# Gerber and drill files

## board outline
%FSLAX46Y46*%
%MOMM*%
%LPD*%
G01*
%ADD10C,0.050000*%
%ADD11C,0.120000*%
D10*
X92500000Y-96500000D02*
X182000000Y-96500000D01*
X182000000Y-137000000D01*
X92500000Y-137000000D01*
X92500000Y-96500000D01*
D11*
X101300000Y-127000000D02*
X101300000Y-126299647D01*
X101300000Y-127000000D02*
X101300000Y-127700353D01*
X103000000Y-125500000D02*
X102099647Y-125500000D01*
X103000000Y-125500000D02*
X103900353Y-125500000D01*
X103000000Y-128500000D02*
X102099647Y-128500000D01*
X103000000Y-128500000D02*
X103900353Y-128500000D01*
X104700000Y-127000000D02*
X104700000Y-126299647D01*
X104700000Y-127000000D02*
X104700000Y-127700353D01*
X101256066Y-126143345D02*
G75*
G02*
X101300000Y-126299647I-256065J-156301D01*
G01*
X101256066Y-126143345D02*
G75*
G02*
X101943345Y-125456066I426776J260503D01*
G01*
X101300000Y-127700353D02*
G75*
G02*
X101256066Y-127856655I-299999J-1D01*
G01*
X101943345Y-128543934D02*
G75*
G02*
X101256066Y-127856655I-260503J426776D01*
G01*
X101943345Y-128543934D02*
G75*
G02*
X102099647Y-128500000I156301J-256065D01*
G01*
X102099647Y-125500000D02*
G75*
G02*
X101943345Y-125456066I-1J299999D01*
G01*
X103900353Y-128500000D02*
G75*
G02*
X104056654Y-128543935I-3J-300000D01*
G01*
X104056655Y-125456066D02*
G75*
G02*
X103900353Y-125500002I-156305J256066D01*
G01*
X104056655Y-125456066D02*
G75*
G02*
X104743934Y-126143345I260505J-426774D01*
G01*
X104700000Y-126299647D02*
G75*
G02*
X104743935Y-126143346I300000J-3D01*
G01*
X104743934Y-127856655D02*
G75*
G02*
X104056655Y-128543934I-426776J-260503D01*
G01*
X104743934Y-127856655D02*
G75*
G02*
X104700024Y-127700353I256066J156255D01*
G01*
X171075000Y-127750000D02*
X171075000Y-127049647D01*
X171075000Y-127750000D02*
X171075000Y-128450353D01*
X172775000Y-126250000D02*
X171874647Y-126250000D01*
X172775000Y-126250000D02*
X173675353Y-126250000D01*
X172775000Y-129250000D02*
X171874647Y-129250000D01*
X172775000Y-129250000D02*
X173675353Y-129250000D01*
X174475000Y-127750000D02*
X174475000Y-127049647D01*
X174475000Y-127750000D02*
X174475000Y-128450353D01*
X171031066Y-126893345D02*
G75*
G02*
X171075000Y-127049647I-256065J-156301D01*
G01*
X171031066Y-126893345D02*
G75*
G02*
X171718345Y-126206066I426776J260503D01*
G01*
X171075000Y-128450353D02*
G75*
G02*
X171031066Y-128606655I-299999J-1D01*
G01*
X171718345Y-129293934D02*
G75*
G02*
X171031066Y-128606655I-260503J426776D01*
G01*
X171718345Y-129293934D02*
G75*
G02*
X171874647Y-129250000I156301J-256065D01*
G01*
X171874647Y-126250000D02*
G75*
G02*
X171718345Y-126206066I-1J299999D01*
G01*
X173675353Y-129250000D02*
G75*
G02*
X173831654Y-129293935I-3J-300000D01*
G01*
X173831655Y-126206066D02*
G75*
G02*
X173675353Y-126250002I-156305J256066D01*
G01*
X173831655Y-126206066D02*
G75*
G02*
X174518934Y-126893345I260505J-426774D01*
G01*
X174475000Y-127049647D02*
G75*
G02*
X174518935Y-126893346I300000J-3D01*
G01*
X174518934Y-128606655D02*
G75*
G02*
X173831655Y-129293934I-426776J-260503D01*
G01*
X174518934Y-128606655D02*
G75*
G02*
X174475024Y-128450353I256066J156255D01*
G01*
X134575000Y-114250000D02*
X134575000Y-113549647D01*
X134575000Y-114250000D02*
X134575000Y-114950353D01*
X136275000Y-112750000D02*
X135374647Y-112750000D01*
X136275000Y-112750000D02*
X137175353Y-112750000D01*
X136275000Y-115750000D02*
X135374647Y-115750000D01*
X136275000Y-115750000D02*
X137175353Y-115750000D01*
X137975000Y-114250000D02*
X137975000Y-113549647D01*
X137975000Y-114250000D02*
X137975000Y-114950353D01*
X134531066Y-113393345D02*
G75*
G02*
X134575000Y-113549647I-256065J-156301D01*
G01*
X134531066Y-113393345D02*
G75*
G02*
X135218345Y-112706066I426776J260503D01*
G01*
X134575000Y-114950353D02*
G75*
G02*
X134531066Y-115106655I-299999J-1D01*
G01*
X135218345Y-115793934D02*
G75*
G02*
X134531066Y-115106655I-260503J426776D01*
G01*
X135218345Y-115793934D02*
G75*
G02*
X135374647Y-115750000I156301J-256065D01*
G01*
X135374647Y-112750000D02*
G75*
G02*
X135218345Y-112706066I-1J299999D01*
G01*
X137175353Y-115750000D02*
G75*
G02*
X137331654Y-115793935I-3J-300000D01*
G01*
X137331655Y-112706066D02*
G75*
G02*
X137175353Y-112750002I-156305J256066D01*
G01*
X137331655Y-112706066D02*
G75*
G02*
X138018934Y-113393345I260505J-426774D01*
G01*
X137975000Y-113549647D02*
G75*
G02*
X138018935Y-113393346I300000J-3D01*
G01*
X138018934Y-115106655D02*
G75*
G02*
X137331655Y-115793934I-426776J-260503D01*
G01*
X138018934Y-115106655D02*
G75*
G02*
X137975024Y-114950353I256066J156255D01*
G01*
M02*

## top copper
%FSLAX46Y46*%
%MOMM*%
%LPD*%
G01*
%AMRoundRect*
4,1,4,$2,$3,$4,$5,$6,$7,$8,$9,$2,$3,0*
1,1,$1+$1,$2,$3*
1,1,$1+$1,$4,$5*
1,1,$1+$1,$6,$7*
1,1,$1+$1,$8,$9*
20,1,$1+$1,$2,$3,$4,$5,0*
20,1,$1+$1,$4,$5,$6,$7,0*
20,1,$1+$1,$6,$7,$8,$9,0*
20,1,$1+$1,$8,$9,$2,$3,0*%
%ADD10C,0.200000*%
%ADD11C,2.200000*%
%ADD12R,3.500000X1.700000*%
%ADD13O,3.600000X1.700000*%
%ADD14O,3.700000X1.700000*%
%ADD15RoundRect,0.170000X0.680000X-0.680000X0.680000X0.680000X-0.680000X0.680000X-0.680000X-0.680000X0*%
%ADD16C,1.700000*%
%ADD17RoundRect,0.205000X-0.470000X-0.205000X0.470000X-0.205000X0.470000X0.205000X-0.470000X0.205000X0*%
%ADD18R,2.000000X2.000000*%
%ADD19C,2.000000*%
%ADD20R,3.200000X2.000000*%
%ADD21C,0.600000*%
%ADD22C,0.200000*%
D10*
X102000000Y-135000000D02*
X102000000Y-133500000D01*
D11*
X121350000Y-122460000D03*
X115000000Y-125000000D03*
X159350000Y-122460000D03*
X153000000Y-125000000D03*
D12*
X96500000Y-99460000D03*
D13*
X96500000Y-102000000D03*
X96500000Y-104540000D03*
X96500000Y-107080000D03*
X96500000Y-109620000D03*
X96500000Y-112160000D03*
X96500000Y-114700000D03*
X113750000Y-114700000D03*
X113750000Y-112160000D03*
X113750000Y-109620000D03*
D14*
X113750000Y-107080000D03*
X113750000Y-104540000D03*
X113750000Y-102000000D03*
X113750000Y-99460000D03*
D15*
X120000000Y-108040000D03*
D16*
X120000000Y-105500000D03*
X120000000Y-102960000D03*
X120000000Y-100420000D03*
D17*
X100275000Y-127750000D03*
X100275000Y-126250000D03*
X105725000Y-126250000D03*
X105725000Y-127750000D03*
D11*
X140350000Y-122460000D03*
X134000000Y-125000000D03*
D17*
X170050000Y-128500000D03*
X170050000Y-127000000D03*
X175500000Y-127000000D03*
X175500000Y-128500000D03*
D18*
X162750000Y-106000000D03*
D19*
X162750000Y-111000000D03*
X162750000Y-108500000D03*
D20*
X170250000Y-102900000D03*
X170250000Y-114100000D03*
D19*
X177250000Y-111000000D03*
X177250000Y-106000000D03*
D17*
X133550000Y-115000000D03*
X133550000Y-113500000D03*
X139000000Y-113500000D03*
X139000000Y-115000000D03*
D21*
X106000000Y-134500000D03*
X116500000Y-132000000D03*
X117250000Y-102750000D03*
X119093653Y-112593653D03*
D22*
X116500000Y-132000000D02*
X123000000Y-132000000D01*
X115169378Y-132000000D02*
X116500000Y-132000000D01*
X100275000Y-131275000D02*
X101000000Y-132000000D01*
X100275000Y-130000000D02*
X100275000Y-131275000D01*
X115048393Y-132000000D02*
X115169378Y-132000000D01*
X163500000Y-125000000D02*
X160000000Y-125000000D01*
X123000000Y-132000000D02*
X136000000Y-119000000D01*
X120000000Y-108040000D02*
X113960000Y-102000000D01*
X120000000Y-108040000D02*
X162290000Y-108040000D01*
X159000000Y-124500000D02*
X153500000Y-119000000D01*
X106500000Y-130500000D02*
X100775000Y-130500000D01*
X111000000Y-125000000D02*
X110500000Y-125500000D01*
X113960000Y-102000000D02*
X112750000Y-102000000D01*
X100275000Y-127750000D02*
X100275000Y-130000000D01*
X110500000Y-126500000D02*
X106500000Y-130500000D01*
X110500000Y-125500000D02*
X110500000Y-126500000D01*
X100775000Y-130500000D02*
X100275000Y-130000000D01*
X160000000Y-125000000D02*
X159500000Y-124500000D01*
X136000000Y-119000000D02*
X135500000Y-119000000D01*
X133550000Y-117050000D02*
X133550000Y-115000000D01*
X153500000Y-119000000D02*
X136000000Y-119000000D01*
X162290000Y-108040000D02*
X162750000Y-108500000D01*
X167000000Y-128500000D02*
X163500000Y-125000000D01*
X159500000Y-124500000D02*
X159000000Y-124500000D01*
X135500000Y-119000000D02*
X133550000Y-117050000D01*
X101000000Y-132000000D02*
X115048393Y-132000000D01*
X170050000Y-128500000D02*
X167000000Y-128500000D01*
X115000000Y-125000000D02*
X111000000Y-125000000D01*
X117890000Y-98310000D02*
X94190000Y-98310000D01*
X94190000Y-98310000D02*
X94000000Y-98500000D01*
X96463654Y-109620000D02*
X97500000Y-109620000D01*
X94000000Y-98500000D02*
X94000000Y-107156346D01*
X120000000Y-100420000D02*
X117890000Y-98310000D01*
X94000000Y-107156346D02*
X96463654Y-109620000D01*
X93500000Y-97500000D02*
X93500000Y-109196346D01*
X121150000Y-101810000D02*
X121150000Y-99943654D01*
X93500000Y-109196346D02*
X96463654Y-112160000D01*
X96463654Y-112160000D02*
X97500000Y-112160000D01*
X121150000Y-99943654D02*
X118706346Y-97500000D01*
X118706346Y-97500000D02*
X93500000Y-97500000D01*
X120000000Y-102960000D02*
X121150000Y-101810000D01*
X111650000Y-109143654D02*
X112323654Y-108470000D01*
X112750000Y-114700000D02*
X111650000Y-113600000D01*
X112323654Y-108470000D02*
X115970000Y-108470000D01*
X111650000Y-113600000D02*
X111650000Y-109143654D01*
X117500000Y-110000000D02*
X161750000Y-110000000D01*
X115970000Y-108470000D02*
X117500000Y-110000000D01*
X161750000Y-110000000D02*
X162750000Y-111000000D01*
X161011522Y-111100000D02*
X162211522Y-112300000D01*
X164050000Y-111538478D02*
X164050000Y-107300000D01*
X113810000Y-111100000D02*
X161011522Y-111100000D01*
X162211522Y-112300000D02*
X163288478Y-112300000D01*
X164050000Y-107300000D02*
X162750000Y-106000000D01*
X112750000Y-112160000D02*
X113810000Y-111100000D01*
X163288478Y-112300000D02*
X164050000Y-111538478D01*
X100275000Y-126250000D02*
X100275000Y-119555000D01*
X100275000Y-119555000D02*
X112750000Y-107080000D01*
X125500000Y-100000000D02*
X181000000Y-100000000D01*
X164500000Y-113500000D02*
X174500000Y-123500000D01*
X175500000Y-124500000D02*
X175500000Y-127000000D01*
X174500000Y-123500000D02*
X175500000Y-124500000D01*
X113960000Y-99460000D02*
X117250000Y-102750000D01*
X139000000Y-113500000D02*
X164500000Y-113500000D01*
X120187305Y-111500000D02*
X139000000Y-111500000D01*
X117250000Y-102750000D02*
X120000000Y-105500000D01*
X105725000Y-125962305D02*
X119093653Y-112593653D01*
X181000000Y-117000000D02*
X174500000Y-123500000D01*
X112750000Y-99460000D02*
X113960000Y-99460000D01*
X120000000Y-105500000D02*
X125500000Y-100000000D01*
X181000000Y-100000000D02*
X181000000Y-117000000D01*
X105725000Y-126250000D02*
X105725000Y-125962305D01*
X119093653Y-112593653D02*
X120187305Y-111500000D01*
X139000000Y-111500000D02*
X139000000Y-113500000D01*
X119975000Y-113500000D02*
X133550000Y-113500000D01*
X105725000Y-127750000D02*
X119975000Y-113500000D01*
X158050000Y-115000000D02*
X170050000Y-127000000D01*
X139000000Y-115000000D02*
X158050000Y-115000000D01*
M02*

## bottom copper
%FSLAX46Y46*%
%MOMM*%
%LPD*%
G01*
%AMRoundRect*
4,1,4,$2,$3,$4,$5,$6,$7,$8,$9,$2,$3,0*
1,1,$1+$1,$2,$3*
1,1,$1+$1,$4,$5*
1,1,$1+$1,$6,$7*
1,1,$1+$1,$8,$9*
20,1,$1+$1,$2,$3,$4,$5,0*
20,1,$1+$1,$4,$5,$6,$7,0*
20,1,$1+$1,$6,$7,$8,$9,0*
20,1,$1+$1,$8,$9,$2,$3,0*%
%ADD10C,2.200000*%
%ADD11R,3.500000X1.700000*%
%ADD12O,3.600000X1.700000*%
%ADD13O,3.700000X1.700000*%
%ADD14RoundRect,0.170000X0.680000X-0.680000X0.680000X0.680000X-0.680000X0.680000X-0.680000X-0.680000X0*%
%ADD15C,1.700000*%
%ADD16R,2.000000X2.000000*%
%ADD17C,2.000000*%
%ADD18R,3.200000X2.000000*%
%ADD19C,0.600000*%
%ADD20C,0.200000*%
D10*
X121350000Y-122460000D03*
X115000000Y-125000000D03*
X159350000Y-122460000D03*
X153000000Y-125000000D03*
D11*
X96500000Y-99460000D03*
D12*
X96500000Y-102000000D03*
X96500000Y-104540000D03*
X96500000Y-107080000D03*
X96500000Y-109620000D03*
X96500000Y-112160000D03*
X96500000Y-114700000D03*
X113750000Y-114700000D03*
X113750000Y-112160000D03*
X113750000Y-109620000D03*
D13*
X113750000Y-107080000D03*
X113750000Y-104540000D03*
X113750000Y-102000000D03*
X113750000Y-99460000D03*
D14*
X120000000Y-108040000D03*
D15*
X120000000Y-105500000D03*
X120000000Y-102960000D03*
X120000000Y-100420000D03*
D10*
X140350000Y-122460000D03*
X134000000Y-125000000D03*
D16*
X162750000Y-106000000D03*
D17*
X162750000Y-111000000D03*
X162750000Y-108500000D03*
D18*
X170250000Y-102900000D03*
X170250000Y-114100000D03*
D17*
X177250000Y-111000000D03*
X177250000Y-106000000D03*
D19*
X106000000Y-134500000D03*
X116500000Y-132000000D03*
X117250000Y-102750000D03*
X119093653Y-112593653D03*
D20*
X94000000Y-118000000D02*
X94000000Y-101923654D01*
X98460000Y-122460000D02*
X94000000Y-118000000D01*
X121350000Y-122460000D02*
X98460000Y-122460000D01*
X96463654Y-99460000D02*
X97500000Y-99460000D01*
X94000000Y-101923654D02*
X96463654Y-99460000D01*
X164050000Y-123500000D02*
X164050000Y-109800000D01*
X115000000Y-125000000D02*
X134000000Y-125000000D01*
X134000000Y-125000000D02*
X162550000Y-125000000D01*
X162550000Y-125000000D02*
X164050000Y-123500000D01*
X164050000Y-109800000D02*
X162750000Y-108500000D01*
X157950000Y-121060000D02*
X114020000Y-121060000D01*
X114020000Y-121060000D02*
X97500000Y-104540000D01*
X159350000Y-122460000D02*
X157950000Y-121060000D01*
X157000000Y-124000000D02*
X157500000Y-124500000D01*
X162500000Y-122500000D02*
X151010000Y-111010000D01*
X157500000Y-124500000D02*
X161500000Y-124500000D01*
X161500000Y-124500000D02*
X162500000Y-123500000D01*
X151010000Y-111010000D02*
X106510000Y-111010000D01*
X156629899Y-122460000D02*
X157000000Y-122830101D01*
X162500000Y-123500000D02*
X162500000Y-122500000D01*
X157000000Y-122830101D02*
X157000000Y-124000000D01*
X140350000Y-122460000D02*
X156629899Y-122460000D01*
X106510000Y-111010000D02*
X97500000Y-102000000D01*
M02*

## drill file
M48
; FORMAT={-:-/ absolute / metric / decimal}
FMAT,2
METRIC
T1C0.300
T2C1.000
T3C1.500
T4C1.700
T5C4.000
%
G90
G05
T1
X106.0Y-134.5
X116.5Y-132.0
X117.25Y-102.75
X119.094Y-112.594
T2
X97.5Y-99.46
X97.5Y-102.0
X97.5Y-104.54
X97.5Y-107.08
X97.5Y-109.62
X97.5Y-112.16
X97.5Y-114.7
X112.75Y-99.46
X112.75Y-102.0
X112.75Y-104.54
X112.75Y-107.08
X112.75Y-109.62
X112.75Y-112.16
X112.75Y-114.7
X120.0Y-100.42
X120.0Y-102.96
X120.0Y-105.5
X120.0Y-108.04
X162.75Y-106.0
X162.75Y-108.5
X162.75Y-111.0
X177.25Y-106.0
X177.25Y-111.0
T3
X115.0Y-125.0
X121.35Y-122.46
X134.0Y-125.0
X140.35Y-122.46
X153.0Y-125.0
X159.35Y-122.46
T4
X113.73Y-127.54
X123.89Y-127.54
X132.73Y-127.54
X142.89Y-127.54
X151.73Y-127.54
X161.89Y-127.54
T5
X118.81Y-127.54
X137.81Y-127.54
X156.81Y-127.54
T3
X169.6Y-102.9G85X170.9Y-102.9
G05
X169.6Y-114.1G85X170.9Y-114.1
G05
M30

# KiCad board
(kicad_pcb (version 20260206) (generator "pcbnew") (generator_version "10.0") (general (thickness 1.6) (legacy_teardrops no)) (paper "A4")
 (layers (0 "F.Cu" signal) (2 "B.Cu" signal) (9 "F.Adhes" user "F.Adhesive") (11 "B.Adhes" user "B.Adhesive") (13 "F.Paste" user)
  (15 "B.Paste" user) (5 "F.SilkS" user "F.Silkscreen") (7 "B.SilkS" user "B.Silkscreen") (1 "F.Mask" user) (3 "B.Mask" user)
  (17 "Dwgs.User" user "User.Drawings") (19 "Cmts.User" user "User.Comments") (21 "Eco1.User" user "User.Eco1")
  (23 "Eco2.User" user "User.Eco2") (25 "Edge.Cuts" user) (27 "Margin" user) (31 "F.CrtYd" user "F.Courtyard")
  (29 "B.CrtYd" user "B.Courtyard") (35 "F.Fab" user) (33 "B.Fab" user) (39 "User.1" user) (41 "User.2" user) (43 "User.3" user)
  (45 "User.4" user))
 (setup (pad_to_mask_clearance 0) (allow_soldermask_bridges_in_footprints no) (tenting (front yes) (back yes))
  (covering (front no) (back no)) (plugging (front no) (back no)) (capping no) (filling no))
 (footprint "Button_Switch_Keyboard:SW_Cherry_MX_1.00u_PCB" (layer "F.Cu") (at 121.35 122.46)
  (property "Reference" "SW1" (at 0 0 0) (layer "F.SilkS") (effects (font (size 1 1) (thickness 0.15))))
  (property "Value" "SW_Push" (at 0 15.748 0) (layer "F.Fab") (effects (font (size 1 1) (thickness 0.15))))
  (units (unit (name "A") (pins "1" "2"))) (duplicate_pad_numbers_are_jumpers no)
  (pad "" np_thru_hole circle (at -7.62 5.08) (size 1.7 1.7) (drill 1.7) (layers "*.Cu" "*.Mask"))
  (pad "" np_thru_hole circle (at -2.54 5.08) (size 4 4) (drill 4) (layers "*.Cu" "*.Mask"))
  (pad "" np_thru_hole circle (at 2.54 5.08) (size 1.7 1.7) (drill 1.7) (layers "*.Cu" "*.Mask"))
  (pad "1" thru_hole circle (at 0 0) (size 2.2 2.2) (drill 1.5) (layers "*.Cu" "*.Mask") (remove_unused_layers no)
   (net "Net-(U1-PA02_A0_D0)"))
  (pad "2" thru_hole circle (at -6.35 2.54) (size 2.2 2.2) (drill 1.5) (layers "*.Cu" "*.Mask") (remove_unused_layers no) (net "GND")))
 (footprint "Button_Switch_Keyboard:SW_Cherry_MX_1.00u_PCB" (layer "F.Cu") (at 159.35 122.46)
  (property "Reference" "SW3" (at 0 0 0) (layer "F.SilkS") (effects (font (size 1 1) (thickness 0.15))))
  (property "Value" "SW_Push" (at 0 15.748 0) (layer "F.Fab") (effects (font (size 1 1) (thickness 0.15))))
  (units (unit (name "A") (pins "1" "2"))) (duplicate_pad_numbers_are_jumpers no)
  (pad "" np_thru_hole circle (at -7.62 5.08) (size 1.7 1.7) (drill 1.7) (layers "*.Cu" "*.Mask"))
  (pad "" np_thru_hole circle (at -2.54 5.08) (size 4 4) (drill 4) (layers "*.Cu" "*.Mask"))
  (pad "" np_thru_hole circle (at 2.54 5.08) (size 1.7 1.7) (drill 1.7) (layers "*.Cu" "*.Mask"))
  (pad "1" thru_hole circle (at 0 0) (size 2.2 2.2) (drill 1.5) (layers "*.Cu" "*.Mask") (remove_unused_layers no)
   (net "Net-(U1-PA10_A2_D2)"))
  (pad "2" thru_hole circle (at -6.35 2.54) (size 2.2 2.2) (drill 1.5) (layers "*.Cu" "*.Mask") (remove_unused_layers no) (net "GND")))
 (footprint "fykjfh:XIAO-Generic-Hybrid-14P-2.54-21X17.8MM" (layer "F.Cu") (at 105.125 107.08)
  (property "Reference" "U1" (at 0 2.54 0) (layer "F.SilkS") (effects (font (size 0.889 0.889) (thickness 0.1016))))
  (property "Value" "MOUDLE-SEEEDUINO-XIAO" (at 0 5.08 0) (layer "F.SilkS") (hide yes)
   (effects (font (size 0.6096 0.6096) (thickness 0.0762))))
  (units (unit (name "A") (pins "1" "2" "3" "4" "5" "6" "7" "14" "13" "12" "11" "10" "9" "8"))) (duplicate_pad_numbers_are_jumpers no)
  (pad "1" thru_hole rect (at -7.625 -7.62) (size 3.5 1.7) (drill 1 (offset -1 0)) (layers "*.Cu" "*.Mask") (remove_unused_layers no)
   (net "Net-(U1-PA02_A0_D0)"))
  (pad "2" thru_hole oval (at -7.625 -5.08) (size 3.6 1.7) (drill 1 (offset -1 0)) (layers "*.Cu" "*.Mask") (remove_unused_layers no)
   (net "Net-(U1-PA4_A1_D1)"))
  (pad "3" thru_hole oval (at -7.625 -2.54) (size 3.6 1.7) (drill 1 (offset -1 0)) (layers "*.Cu" "*.Mask") (remove_unused_layers no)
   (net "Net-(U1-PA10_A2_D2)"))
  (pad "4" thru_hole oval (at -7.625 0) (size 3.6 1.7) (drill 1 (offset -1 0)) (layers "*.Cu" "*.Mask") (remove_unused_layers no)
   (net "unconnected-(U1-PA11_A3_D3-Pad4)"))
  (pad "5" thru_hole oval (at -7.625 2.54) (size 3.6 1.7) (drill 1 (offset -1 0)) (layers "*.Cu" "*.Mask") (remove_unused_layers no)
   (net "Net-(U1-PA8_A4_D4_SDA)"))
  (pad "6" thru_hole oval (at -7.625 5.08 180) (size 3.6 1.7) (drill 1 (offset 1 0)) (layers "*.Cu" "*.Mask") (remove_unused_layers no)
   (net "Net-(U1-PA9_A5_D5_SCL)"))
  (pad "7" thru_hole oval (at -7.625 7.62) (size 3.6 1.7) (drill 1 (offset -1 0)) (layers "*.Cu" "*.Mask") (remove_unused_layers no)
   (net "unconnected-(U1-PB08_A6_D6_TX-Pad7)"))
  (pad "8" thru_hole oval (at 7.625 7.62) (size 3.6 1.7) (drill 1 (offset 1 0)) (layers "*.Cu" "*.Mask") (remove_unused_layers no)
   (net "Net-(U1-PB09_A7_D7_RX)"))
  (pad "9" thru_hole oval (at 7.625 5.08) (size 3.6 1.7) (drill 1 (offset 1 0)) (layers "*.Cu" "*.Mask") (remove_unused_layers no)
   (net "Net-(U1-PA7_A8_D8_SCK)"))
  (pad "10" thru_hole oval (at 7.625 2.54) (size 3.6 1.7) (drill 1 (offset 1 0)) (layers "*.Cu" "*.Mask") (remove_unused_layers no)
   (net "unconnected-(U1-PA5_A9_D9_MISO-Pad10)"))
  (pad "11" thru_hole oval (at 7.625 0) (size 3.7 1.7) (drill 1 (offset 1 0)) (layers "*.Cu" "*.Mask") (remove_unused_layers no)
   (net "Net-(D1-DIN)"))
  (pad "12" thru_hole oval (at 7.625 -2.54) (size 3.7 1.7) (drill 1 (offset 1 0)) (layers "*.Cu" "*.Mask") (remove_unused_layers no)
   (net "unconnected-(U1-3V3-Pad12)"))
  (pad "13" thru_hole oval (at 7.625 -5.08) (size 3.7 1.7) (drill 1 (offset 1 0)) (layers "*.Cu" "*.Mask") (remove_unused_layers no)
   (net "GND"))
  (pad "14" thru_hole oval (at 7.625 -7.62) (size 3.7 1.7) (drill 1 (offset 1 0)) (layers "*.Cu" "*.Mask") (remove_unused_layers no)
   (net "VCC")))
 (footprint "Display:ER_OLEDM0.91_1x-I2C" (layer "F.Cu") (at 120 108.04 90)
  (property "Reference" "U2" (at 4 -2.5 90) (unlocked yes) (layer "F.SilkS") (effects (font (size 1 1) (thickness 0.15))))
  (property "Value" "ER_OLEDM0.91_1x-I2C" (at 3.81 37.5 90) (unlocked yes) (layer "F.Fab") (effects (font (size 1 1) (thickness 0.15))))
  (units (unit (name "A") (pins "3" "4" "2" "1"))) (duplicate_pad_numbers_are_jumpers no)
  (pad "1" thru_hole roundrect (at 0 0 90) (size 1.7 1.7) (drill 1) (layers "*.Cu" "*.Mask") (remove_unused_layers no)
   (roundrect_rratio 0.1) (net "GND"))
  (pad "2" thru_hole circle (at 2.54 0 90) (size 1.7 1.7) (drill 1) (layers "*.Cu" "*.Mask") (remove_unused_layers no) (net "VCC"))
  (pad "3" thru_hole circle (at 5.08 0 90) (size 1.7 1.7) (drill 1) (layers "*.Cu" "*.Mask") (remove_unused_layers no)
   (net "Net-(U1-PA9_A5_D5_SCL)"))
  (pad "4" thru_hole circle (at 7.62 0 90) (size 1.7 1.7) (drill 1) (layers "*.Cu" "*.Mask") (remove_unused_layers no)
   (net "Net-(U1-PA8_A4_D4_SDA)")))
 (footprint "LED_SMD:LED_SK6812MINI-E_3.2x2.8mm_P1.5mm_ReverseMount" (layer "F.Cu") (at 103 127)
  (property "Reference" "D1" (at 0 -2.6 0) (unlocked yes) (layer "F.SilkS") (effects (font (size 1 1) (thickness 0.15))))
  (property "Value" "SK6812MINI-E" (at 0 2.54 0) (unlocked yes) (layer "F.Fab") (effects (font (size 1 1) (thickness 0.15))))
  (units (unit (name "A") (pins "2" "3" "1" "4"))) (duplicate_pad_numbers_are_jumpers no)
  (fp_line (start -1.7 0) (end -1.7 -0.700353) (stroke (width 0.12) (type solid)) (layer "Edge.Cuts"))
  (fp_line (start -1.7 0) (end -1.7 0.700353) (stroke (width 0.12) (type solid)) (layer "Edge.Cuts"))
  (fp_line (start 0 -1.5) (end -0.900353 -1.5) (stroke (width 0.12) (type solid)) (layer "Edge.Cuts"))
  (fp_line (start 0 -1.5) (end 0.900353 -1.5) (stroke (width 0.12) (type solid)) (layer "Edge.Cuts"))
  (fp_line (start 0 1.5) (end -0.900353 1.5) (stroke (width 0.12) (type solid)) (layer "Edge.Cuts"))
  (fp_line (start 0 1.5) (end 0.900353 1.5) (stroke (width 0.12) (type solid)) (layer "Edge.Cuts"))
  (fp_line (start 1.7 0) (end 1.7 -0.700353) (stroke (width 0.12) (type solid)) (layer "Edge.Cuts"))
  (fp_line (start 1.7 0) (end 1.7 0.700353) (stroke (width 0.12) (type solid)) (layer "Edge.Cuts"))
  (fp_arc (start -1.743934 -0.856655) (mid -1.711192 -0.781532) (end -1.7 -0.700353) (stroke (width 0.12) (type solid)) (layer "Edge.Cuts"))
  (fp_arc (start -1.743934 -0.856655) (mid -1.670711 -1.470711) (end -1.056655 -1.543934) (stroke (width 0.12) (type solid))
   (layer "Edge.Cuts"))
  (fp_arc (start -1.7 0.700353) (mid -1.711192 0.781532) (end -1.743934 0.856655) (stroke (width 0.12) (type solid)) (layer "Edge.Cuts"))
  (fp_arc (start -1.056655 1.543934) (mid -1.670711 1.470711) (end -1.743934 0.856655) (stroke (width 0.12) (type solid))
   (layer "Edge.Cuts"))
  (fp_arc (start -1.056655 1.543934) (mid -0.981532 1.511192) (end -0.900353 1.5) (stroke (width 0.12) (type solid)) (layer "Edge.Cuts"))
  (fp_arc (start -0.900353 -1.5) (mid -0.981532 -1.511192) (end -1.056655 -1.543934) (stroke (width 0.12) (type solid)) (layer "Edge.Cuts"))
  (fp_arc (start 0.900353 1.5) (mid 0.981532 1.511192) (end 1.056655 1.543934) (stroke (width 0.12) (type solid)) (layer "Edge.Cuts"))
  (fp_arc (start 1.056655 -1.543934) (mid 0.981532 -1.511192) (end 0.900353 -1.5) (stroke (width 0.12) (type solid)) (layer "Edge.Cuts"))
  (fp_arc (start 1.056655 -1.543934) (mid 1.670711 -1.470711) (end 1.743934 -0.856655) (stroke (width 0.12) (type solid))
   (layer "Edge.Cuts"))
  (fp_arc (start 1.7 -0.700353) (mid 1.711192 -0.781532) (end 1.743934 -0.856655) (stroke (width 0.12) (type solid)) (layer "Edge.Cuts"))
  (fp_arc (start 1.743934 0.856655) (mid 1.670711 1.470711) (end 1.056655 1.543934) (stroke (width 0.12) (type solid)) (layer "Edge.Cuts"))
  (fp_arc (start 1.743934 0.856655) (mid 1.711192 0.781532) (end 1.7 0.700353) (stroke (width 0.12) (type solid)) (layer "Edge.Cuts"))
  (pad "1" smd roundrect (at -2.725 0.75) (size 1.35 0.82) (layers "F.Cu" "F.Mask" "F.Paste") (roundrect_rratio 0.25) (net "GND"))
  (pad "2" smd roundrect (at -2.725 -0.75) (size 1.35 0.82) (layers "F.Cu" "F.Mask" "F.Paste") (roundrect_rratio 0.25) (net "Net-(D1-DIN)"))
  (pad "3" smd roundrect (at 2.725 -0.75) (size 1.35 0.82) (layers "F.Cu" "F.Mask" "F.Paste") (roundrect_rratio 0.25) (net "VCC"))
  (pad "4" smd roundrect (at 2.725 0.75) (size 1.35 0.82) (layers "F.Cu" "F.Mask" "F.Paste") (roundrect_rratio 0.25) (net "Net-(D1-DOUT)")))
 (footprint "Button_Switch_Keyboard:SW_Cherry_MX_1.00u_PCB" (layer "F.Cu") (at 140.35 122.46)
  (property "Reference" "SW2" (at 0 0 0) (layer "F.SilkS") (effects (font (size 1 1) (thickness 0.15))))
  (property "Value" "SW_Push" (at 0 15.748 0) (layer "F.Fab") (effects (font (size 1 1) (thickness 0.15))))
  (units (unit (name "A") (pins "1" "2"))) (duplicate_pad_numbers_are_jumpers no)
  (pad "" np_thru_hole circle (at -7.62 5.08) (size 1.7 1.7) (drill 1.7) (layers "*.Cu" "*.Mask"))
  (pad "" np_thru_hole circle (at -2.54 5.08) (size 4 4) (drill 4) (layers "*.Cu" "*.Mask"))
  (pad "" np_thru_hole circle (at 2.54 5.08) (size 1.7 1.7) (drill 1.7) (layers "*.Cu" "*.Mask"))
  (pad "1" thru_hole circle (at 0 0) (size 2.2 2.2) (drill 1.5) (layers "*.Cu" "*.Mask") (remove_unused_layers no)
   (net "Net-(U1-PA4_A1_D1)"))
  (pad "2" thru_hole circle (at -6.35 2.54) (size 2.2 2.2) (drill 1.5) (layers "*.Cu" "*.Mask") (remove_unused_layers no) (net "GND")))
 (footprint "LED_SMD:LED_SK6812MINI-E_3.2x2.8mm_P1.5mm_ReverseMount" (layer "F.Cu") (at 172.775 127.75)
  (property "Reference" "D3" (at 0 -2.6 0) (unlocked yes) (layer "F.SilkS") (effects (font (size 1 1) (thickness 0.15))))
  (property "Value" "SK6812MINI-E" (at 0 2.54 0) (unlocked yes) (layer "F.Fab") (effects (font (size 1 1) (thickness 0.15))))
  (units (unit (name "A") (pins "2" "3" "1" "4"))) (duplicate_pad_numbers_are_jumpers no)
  (fp_line (start -1.7 0) (end -1.7 -0.700353) (stroke (width 0.12) (type solid)) (layer "Edge.Cuts"))
  (fp_line (start -1.7 0) (end -1.7 0.700353) (stroke (width 0.12) (type solid)) (layer "Edge.Cuts"))
  (fp_line (start 0 -1.5) (end -0.900353 -1.5) (stroke (width 0.12) (type solid)) (layer "Edge.Cuts"))
  (fp_line (start 0 -1.5) (end 0.900353 -1.5) (stroke (width 0.12) (type solid)) (layer "Edge.Cuts"))
  (fp_line (start 0 1.5) (end -0.900353 1.5) (stroke (width 0.12) (type solid)) (layer "Edge.Cuts"))
  (fp_line (start 0 1.5) (end 0.900353 1.5) (stroke (width 0.12) (type solid)) (layer "Edge.Cuts"))
  (fp_line (start 1.7 0) (end 1.7 -0.700353) (stroke (width 0.12) (type solid)) (layer "Edge.Cuts"))
  (fp_line (start 1.7 0) (end 1.7 0.700353) (stroke (width 0.12) (type solid)) (layer "Edge.Cuts"))
  (fp_arc (start -1.743934 -0.856655) (mid -1.711192 -0.781532) (end -1.7 -0.700353) (stroke (width 0.12) (type solid)) (layer "Edge.Cuts"))
  (fp_arc (start -1.743934 -0.856655) (mid -1.670711 -1.470711) (end -1.056655 -1.543934) (stroke (width 0.12) (type solid))
   (layer "Edge.Cuts"))
  (fp_arc (start -1.7 0.700353) (mid -1.711192 0.781532) (end -1.743934 0.856655) (stroke (width 0.12) (type solid)) (layer "Edge.Cuts"))
  (fp_arc (start -1.056655 1.543934) (mid -1.670711 1.470711) (end -1.743934 0.856655) (stroke (width 0.12) (type solid))
   (layer "Edge.Cuts"))
  (fp_arc (start -1.056655 1.543934) (mid -0.981532 1.511192) (end -0.900353 1.5) (stroke (width 0.12) (type solid)) (layer "Edge.Cuts"))
  (fp_arc (start -0.900353 -1.5) (mid -0.981532 -1.511192) (end -1.056655 -1.543934) (stroke (width 0.12) (type solid)) (layer "Edge.Cuts"))
  (fp_arc (start 0.900353 1.5) (mid 0.981532 1.511192) (end 1.056655 1.543934) (stroke (width 0.12) (type solid)) (layer "Edge.Cuts"))
  (fp_arc (start 1.056655 -1.543934) (mid 0.981532 -1.511192) (end 0.900353 -1.5) (stroke (width 0.12) (type solid)) (layer "Edge.Cuts"))
  (fp_arc (start 1.056655 -1.543934) (mid 1.670711 -1.470711) (end 1.743934 -0.856655) (stroke (width 0.12) (type solid))
   (layer "Edge.Cuts"))
  (fp_arc (start 1.7 -0.700353) (mid 1.711192 -0.781532) (end 1.743934 -0.856655) (stroke (width 0.12) (type solid)) (layer "Edge.Cuts"))
  (fp_arc (start 1.743934 0.856655) (mid 1.670711 1.470711) (end 1.056655 1.543934) (stroke (width 0.12) (type solid)) (layer "Edge.Cuts"))
  (fp_arc (start 1.743934 0.856655) (mid 1.711192 0.781532) (end 1.7 0.700353) (stroke (width 0.12) (type solid)) (layer "Edge.Cuts"))
  (pad "1" smd roundrect (at -2.725 0.75) (size 1.35 0.82) (layers "F.Cu" "F.Mask" "F.Paste") (roundrect_rratio 0.25) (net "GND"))
  (pad "2" smd roundrect (at -2.725 -0.75) (size 1.35 0.82) (layers "F.Cu" "F.Mask" "F.Paste") (roundrect_rratio 0.25) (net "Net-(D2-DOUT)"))
  (pad "3" smd roundrect (at 2.725 -0.75) (size 1.35 0.82) (layers "F.Cu" "F.Mask" "F.Paste") (roundrect_rratio 0.25) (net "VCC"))
  (pad "4" smd roundrect (at 2.725 0.75) (size 1.35 0.82) (layers "F.Cu" "F.Mask" "F.Paste") (roundrect_rratio 0.25)
   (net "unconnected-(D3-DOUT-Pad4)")))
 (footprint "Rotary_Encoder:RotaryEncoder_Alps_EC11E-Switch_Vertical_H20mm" (layer "F.Cu") (at 162.75 106)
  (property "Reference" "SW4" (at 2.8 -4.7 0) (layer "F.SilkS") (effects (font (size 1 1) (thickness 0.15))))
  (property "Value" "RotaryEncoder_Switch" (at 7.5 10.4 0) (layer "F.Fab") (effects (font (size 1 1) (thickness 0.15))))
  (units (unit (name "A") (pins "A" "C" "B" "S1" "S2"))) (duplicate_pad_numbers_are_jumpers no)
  (pad "A" thru_hole rect (at 0 0) (size 2 2) (drill 1) (layers "*.Cu" "*.Mask") (remove_unused_layers no) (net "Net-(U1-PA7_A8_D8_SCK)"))
  (pad "B" thru_hole circle (at 0 5) (size 2 2) (drill 1) (layers "*.Cu" "*.Mask") (remove_unused_layers no) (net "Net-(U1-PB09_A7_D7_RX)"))
  (pad "C" thru_hole circle (at 0 2.5) (size 2 2) (drill 1) (layers "*.Cu" "*.Mask") (remove_unused_layers no) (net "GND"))
  (pad "MP" thru_hole rect (at 7.5 -3.1) (size 3.2 2) (drill oval 2.8 1.5) (layers "*.Cu" "*.Mask") (remove_unused_layers no))
  (pad "MP" thru_hole rect (at 7.5 8.1) (size 3.2 2) (drill oval 2.8 1.5) (layers "*.Cu" "*.Mask") (remove_unused_layers no))
  (pad "S1" thru_hole circle (at 14.5 5) (size 2 2) (drill 1) (layers "*.Cu" "*.Mask") (remove_unused_layers no)
   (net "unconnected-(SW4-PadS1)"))
  (pad "S2" thru_hole circle (at 14.5 0) (size 2 2) (drill 1) (layers "*.Cu" "*.Mask") (remove_unused_layers no)
   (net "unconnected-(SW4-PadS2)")))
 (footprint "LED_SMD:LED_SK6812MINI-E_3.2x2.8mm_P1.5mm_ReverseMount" (layer "F.Cu") (at 136.275 114.25)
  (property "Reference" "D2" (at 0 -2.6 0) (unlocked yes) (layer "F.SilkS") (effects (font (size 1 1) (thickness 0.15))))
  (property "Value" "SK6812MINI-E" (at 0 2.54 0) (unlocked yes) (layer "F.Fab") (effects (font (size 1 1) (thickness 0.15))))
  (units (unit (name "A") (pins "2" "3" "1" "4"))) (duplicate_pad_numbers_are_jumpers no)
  (fp_line (start -1.7 0) (end -1.7 -0.700353) (stroke (width 0.12) (type solid)) (layer "Edge.Cuts"))
  (fp_line (start -1.7 0) (end -1.7 0.700353) (stroke (width 0.12) (type solid)) (layer "Edge.Cuts"))
  (fp_line (start 0 -1.5) (end -0.900353 -1.5) (stroke (width 0.12) (type solid)) (layer "Edge.Cuts"))
  (fp_line (start 0 -1.5) (end 0.900353 -1.5) (stroke (width 0.12) (type solid)) (layer "Edge.Cuts"))
  (fp_line (start 0 1.5) (end -0.900353 1.5) (stroke (width 0.12) (type solid)) (layer "Edge.Cuts"))
  (fp_line (start 0 1.5) (end 0.900353 1.5) (stroke (width 0.12) (type solid)) (layer "Edge.Cuts"))
  (fp_line (start 1.7 0) (end 1.7 -0.700353) (stroke (width 0.12) (type solid)) (layer "Edge.Cuts"))
  (fp_line (start 1.7 0) (end 1.7 0.700353) (stroke (width 0.12) (type solid)) (layer "Edge.Cuts"))
  (fp_arc (start -1.743934 -0.856655) (mid -1.711192 -0.781532) (end -1.7 -0.700353) (stroke (width 0.12) (type solid)) (layer "Edge.Cuts"))
  (fp_arc (start -1.743934 -0.856655) (mid -1.670711 -1.470711) (end -1.056655 -1.543934) (stroke (width 0.12) (type solid))
   (layer "Edge.Cuts"))
  (fp_arc (start -1.7 0.700353) (mid -1.711192 0.781532) (end -1.743934 0.856655) (stroke (width 0.12) (type solid)) (layer "Edge.Cuts"))
  (fp_arc (start -1.056655 1.543934) (mid -1.670711 1.470711) (end -1.743934 0.856655) (stroke (width 0.12) (type solid))
   (layer "Edge.Cuts"))
  (fp_arc (start -1.056655 1.543934) (mid -0.981532 1.511192) (end -0.900353 1.5) (stroke (width 0.12) (type solid)) (layer "Edge.Cuts"))
  (fp_arc (start -0.900353 -1.5) (mid -0.981532 -1.511192) (end -1.056655 -1.543934) (stroke (width 0.12) (type solid)) (layer "Edge.Cuts"))
  (fp_arc (start 0.900353 1.5) (mid 0.981532 1.511192) (end 1.056655 1.543934) (stroke (width 0.12) (type solid)) (layer "Edge.Cuts"))
  (fp_arc (start 1.056655 -1.543934) (mid 0.981532 -1.511192) (end 0.900353 -1.5) (stroke (width 0.12) (type solid)) (layer "Edge.Cuts"))
  (fp_arc (start 1.056655 -1.543934) (mid 1.670711 -1.470711) (end 1.743934 -0.856655) (stroke (width 0.12) (type solid))
   (layer "Edge.Cuts"))
  (fp_arc (start 1.7 -0.700353) (mid 1.711192 -0.781532) (end 1.743934 -0.856655) (stroke (width 0.12) (type solid)) (layer "Edge.Cuts"))
  (fp_arc (start 1.743934 0.856655) (mid 1.670711 1.470711) (end 1.056655 1.543934) (stroke (width 0.12) (type solid)) (layer "Edge.Cuts"))
  (fp_arc (start 1.743934 0.856655) (mid 1.711192 0.781532) (end 1.7 0.700353) (stroke (width 0.12) (type solid)) (layer "Edge.Cuts"))
  (pad "1" smd roundrect (at -2.725 0.75) (size 1.35 0.82) (layers "F.Cu" "F.Mask" "F.Paste") (roundrect_rratio 0.25) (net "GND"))
  (pad "2" smd roundrect (at -2.725 -0.75) (size 1.35 0.82) (layers "F.Cu" "F.Mask" "F.Paste") (roundrect_rratio 0.25) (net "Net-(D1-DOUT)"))
  (pad "3" smd roundrect (at 2.725 -0.75) (size 1.35 0.82) (layers "F.Cu" "F.Mask" "F.Paste") (roundrect_rratio 0.25) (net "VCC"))
  (pad "4" smd roundrect (at 2.725 0.75) (size 1.35 0.82) (layers "F.Cu" "F.Mask" "F.Paste") (roundrect_rratio 0.25) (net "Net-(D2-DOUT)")))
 (gr_line (start 102 135) (end 102 133.5) (stroke (width 0.2) (type default)) (layer "F.Cu"))
 (gr_rect (start 92.5 96.5) (end 182 137) (stroke (width 0.05) (type default)) (fill no) (layer "Edge.Cuts"))
 (via (at 106 134.5) (size 0.6) (drill 0.3) (layers "F.Cu" "B.Cu") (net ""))
 (segment (start 94 118) (end 94 101.923654) (width 0.2) (layer "B.Cu") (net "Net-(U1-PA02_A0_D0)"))
 (segment (start 98.46 122.46) (end 94 118) (width 0.2) (layer "B.Cu") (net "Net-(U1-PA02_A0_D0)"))
 (segment (start 121.35 122.46) (end 98.46 122.46) (width 0.2) (layer "B.Cu") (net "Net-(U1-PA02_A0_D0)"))
 (segment (start 96.463654 99.46) (end 97.5 99.46) (width 0.2) (layer "B.Cu") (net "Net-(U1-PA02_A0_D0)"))
 (segment (start 94 101.923654) (end 96.463654 99.46) (width 0.2) (layer "B.Cu") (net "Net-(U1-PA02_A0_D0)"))
 (segment (start 116.5 132) (end 123 132) (width 0.2) (layer "F.Cu") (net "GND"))
 (segment (start 115.169378 132) (end 116.5 132) (width 0.2) (layer "F.Cu") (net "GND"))
 (segment (start 100.275 131.275) (end 101 132) (width 0.2) (layer "F.Cu") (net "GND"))
 (segment (start 100.275 130) (end 100.275 131.275) (width 0.2) (layer "F.Cu") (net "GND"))
 (segment (start 115.048393 132) (end 115.169378 132) (width 0.2) (layer "F.Cu") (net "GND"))
 (segment (start 163.5 125) (end 160 125) (width 0.2) (layer "F.Cu") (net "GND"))
 (segment (start 123 132) (end 136 119) (width 0.2) (layer "F.Cu") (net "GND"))
 (segment (start 120 108.04) (end 113.96 102) (width 0.2) (layer "F.Cu") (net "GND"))
 (segment (start 120 108.04) (end 162.29 108.04) (width 0.2) (layer "F.Cu") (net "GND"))
 (segment (start 159 124.5) (end 153.5 119) (width 0.2) (layer "F.Cu") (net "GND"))
 (segment (start 106.5 130.5) (end 100.775 130.5) (width 0.2) (layer "F.Cu") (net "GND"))
 (segment (start 111 125) (end 110.5 125.5) (width 0.2) (layer "F.Cu") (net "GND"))
 (segment (start 113.96 102) (end 112.75 102) (width 0.2) (layer "F.Cu") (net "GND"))
 (segment (start 100.275 127.75) (end 100.275 130) (width 0.2) (layer "F.Cu") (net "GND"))
 (segment (start 110.5 126.5) (end 106.5 130.5) (width 0.2) (layer "F.Cu") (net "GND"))
 (segment (start 110.5 125.5) (end 110.5 126.5) (width 0.2) (layer "F.Cu") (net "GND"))
 (segment (start 100.775 130.5) (end 100.275 130) (width 0.2) (layer "F.Cu") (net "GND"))
 (segment (start 160 125) (end 159.5 124.5) (width 0.2) (layer "F.Cu") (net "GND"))
 (segment (start 136 119) (end 135.5 119) (width 0.2) (layer "F.Cu") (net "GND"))
 (segment (start 133.55 117.05) (end 133.55 115) (width 0.2) (layer "F.Cu") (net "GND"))
 (segment (start 153.5 119) (end 136 119) (width 0.2) (layer "F.Cu") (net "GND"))
 (segment (start 162.29 108.04) (end 162.75 108.5) (width 0.2) (layer "F.Cu") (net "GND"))
 (segment (start 167 128.5) (end 163.5 125) (width 0.2) (layer "F.Cu") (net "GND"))
 (segment (start 159.5 124.5) (end 159 124.5) (width 0.2) (layer "F.Cu") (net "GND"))
 (segment (start 135.5 119) (end 133.55 117.05) (width 0.2) (layer "F.Cu") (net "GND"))
 (segment (start 101 132) (end 115.048393 132) (width 0.2) (layer "F.Cu") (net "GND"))
 (segment (start 170.05 128.5) (end 167 128.5) (width 0.2) (layer "F.Cu") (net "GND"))
 (segment (start 115 125) (end 111 125) (width 0.2) (layer "F.Cu") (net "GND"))
 (via (at 116.5 132) (size 0.6) (drill 0.3) (layers "F.Cu" "B.Cu") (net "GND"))
 (segment (start 164.05 123.5) (end 164.05 109.8) (width 0.2) (layer "B.Cu") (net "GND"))
 (segment (start 115 125) (end 134 125) (width 0.2) (layer "B.Cu") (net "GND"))
 (segment (start 134 125) (end 162.55 125) (width 0.2) (layer "B.Cu") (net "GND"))
 (segment (start 162.55 125) (end 164.05 123.5) (width 0.2) (layer "B.Cu") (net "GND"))
 (segment (start 164.05 109.8) (end 162.75 108.5) (width 0.2) (layer "B.Cu") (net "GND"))
 (segment (start 157.95 121.06) (end 114.02 121.06) (width 0.2) (layer "B.Cu") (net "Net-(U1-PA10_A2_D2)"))
 (segment (start 114.02 121.06) (end 97.5 104.54) (width 0.2) (layer "B.Cu") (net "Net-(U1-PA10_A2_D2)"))
 (segment (start 159.35 122.46) (end 157.95 121.06) (width 0.2) (layer "B.Cu") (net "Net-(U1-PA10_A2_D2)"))
 (segment (start 157 124) (end 157.5 124.5) (width 0.2) (layer "B.Cu") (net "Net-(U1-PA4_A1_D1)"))
 (segment (start 162.5 122.5) (end 151.01 111.01) (width 0.2) (layer "B.Cu") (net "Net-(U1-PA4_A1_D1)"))
 (segment (start 157.5 124.5) (end 161.5 124.5) (width 0.2) (layer "B.Cu") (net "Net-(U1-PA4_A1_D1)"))
 (segment (start 161.5 124.5) (end 162.5 123.5) (width 0.2) (layer "B.Cu") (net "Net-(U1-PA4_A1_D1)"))
 (segment (start 151.01 111.01) (end 106.51 111.01) (width 0.2) (layer "B.Cu") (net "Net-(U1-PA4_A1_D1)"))
 (segment (start 156.629899 122.46) (end 157 122.830101) (width 0.2) (layer "B.Cu") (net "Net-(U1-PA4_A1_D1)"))
 (segment (start 162.5 123.5) (end 162.5 122.5) (width 0.2) (layer "B.Cu") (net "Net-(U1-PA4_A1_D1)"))
 (segment (start 157 122.830101) (end 157 124) (width 0.2) (layer "B.Cu") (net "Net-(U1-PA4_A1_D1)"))
 (segment (start 140.35 122.46) (end 156.629899 122.46) (width 0.2) (layer "B.Cu") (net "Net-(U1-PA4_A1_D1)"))
 (segment (start 106.51 111.01) (end 97.5 102) (width 0.2) (layer "B.Cu") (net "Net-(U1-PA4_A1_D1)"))
 (segment (start 117.89 98.31) (end 94.19 98.31) (width 0.2) (layer "F.Cu") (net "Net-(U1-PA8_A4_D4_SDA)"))
 (segment (start 94.19 98.31) (end 94 98.5) (width 0.2) (layer "F.Cu") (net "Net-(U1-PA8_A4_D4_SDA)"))
 (segment (start 96.463654 109.62) (end 97.5 109.62) (width 0.2) (layer "F.Cu") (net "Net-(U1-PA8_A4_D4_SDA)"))
 (segment (start 94 98.5) (end 94 107.156346) (width 0.2) (layer "F.Cu") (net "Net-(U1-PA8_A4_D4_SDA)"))
 (segment (start 120 100.42) (end 117.89 98.31) (width 0.2) (layer "F.Cu") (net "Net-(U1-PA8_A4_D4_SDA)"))
 (segment (start 94 107.156346) (end 96.463654 109.62) (width 0.2) (layer "F.Cu") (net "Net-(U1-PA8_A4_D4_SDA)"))
 (segment (start 93.5 97.5) (end 93.5 109.196346) (width 0.2) (layer "F.Cu") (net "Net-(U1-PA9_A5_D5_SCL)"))
 (segment (start 121.15 101.81) (end 121.15 99.943654) (width 0.2) (layer "F.Cu") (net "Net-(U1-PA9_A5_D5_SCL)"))
 (segment (start 93.5 109.196346) (end 96.463654 112.16) (width 0.2) (layer "F.Cu") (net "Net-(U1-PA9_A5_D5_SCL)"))
 (segment (start 96.463654 112.16) (end 97.5 112.16) (width 0.2) (layer "F.Cu") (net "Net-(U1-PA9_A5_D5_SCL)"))
 (segment (start 121.15 99.943654) (end 118.706346 97.5) (width 0.2) (layer "F.Cu") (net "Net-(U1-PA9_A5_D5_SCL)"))
 (segment (start 118.706346 97.5) (end 93.5 97.5) (width 0.2) (layer "F.Cu") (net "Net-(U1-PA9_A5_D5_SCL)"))
 (segment (start 120 102.96) (end 121.15 101.81) (width 0.2) (layer "F.Cu") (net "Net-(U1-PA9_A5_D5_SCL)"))
 (segment (start 111.65 109.143654) (end 112.323654 108.47) (width 0.2) (layer "F.Cu") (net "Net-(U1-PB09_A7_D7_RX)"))
 (segment (start 112.75 114.7) (end 111.65 113.6) (width 0.2) (layer "F.Cu") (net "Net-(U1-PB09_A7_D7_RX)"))
 (segment (start 112.323654 108.47) (end 115.97 108.47) (width 0.2) (layer "F.Cu") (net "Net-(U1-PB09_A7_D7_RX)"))
 (segment (start 111.65 113.6) (end 111.65 109.143654) (width 0.2) (layer "F.Cu") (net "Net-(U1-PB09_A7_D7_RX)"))
 (segment (start 117.5 110) (end 161.75 110) (width 0.2) (layer "F.Cu") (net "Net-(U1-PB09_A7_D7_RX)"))
 (segment (start 115.97 108.47) (end 117.5 110) (width 0.2) (layer "F.Cu") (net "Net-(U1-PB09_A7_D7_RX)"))
 (segment (start 161.75 110) (end 162.75 111) (width 0.2) (layer "F.Cu") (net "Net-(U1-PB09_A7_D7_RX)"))
 (segment (start 161.011522 111.1) (end 162.211522 112.3) (width 0.2) (layer "F.Cu") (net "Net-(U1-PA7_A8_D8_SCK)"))
 (segment (start 164.05 111.538478) (end 164.05 107.3) (width 0.2) (layer "F.Cu") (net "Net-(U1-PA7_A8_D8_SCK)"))
 (segment (start 113.81 111.1) (end 161.011522 111.1) (width 0.2) (layer "F.Cu") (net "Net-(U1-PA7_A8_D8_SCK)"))
 (segment (start 162.211522 112.3) (end 163.288478 112.3) (width 0.2) (layer "F.Cu") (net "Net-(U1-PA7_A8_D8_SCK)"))
 (segment (start 164.05 107.3) (end 162.75 106) (width 0.2) (layer "F.Cu") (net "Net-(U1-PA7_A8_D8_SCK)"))
 (segment (start 112.75 112.16) (end 113.81 111.1) (width 0.2) (layer "F.Cu") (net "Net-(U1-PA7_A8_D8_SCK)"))
 (segment (start 163.288478 112.3) (end 164.05 111.538478) (width 0.2) (layer "F.Cu") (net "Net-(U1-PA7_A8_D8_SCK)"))
 (segment (start 100.275 126.25) (end 100.275 119.555) (width 0.2) (layer "F.Cu") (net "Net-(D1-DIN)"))
 (segment (start 100.275 119.555) (end 112.75 107.08) (width 0.2) (layer "F.Cu") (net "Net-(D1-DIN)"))
 (segment (start 125.5 100) (end 181 100) (width 0.2) (layer "F.Cu") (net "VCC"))
 (segment (start 164.5 113.5) (end 174.5 123.5) (width 0.2) (layer "F.Cu") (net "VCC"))
 (segment (start 175.5 124.5) (end 175.5 127) (width 0.2) (layer "F.Cu") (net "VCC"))
 (segment (start 174.5 123.5) (end 175.5 124.5) (width 0.2) (layer "F.Cu") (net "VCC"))
 (segment (start 113.96 99.46) (end 117.25 102.75) (width 0.2) (layer "F.Cu") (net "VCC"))
 (segment (start 139 113.5) (end 164.5 113.5) (width 0.2) (layer "F.Cu") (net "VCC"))
 (segment (start 120.187305 111.5) (end 139 111.5) (width 0.2) (layer "F.Cu") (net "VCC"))
 (segment (start 117.25 102.75) (end 120 105.5) (width 0.2) (layer "F.Cu") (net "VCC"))
 (segment (start 105.725 125.962305) (end 119.093653 112.593653) (width 0.2) (layer "F.Cu") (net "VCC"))
 (segment (start 181 117) (end 174.5 123.5) (width 0.2) (layer "F.Cu") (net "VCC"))
 (segment (start 112.75 99.46) (end 113.96 99.46) (width 0.2) (layer "F.Cu") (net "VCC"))
 (segment (start 120 105.5) (end 125.5 100) (width 0.2) (layer "F.Cu") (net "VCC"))
 (segment (start 181 100) (end 181 117) (width 0.2) (layer "F.Cu") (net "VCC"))
 (segment (start 105.725 126.25) (end 105.725 125.962305) (width 0.2) (layer "F.Cu") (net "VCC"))
 (segment (start 119.093653 112.593653) (end 120.187305 111.5) (width 0.2) (layer "F.Cu") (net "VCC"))
 (segment (start 139 111.5) (end 139 113.5) (width 0.2) (layer "F.Cu") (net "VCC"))
 (via (at 117.25 102.75) (size 0.6) (drill 0.3) (layers "F.Cu" "B.Cu") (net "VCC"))
 (via (at 119.093653 112.593653) (size 0.6) (drill 0.3) (layers "F.Cu" "B.Cu") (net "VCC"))
 (segment (start 119.975 113.5) (end 133.55 113.5) (width 0.2) (layer "F.Cu") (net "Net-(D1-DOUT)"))
 (segment (start 105.725 127.75) (end 119.975 113.5) (width 0.2) (layer "F.Cu") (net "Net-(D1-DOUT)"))
 (segment (start 158.05 115) (end 170.05 127) (width 0.2) (layer "F.Cu") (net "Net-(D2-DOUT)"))
 (segment (start 139 115) (end 158.05 115) (width 0.2) (layer "F.Cu") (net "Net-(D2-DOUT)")))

